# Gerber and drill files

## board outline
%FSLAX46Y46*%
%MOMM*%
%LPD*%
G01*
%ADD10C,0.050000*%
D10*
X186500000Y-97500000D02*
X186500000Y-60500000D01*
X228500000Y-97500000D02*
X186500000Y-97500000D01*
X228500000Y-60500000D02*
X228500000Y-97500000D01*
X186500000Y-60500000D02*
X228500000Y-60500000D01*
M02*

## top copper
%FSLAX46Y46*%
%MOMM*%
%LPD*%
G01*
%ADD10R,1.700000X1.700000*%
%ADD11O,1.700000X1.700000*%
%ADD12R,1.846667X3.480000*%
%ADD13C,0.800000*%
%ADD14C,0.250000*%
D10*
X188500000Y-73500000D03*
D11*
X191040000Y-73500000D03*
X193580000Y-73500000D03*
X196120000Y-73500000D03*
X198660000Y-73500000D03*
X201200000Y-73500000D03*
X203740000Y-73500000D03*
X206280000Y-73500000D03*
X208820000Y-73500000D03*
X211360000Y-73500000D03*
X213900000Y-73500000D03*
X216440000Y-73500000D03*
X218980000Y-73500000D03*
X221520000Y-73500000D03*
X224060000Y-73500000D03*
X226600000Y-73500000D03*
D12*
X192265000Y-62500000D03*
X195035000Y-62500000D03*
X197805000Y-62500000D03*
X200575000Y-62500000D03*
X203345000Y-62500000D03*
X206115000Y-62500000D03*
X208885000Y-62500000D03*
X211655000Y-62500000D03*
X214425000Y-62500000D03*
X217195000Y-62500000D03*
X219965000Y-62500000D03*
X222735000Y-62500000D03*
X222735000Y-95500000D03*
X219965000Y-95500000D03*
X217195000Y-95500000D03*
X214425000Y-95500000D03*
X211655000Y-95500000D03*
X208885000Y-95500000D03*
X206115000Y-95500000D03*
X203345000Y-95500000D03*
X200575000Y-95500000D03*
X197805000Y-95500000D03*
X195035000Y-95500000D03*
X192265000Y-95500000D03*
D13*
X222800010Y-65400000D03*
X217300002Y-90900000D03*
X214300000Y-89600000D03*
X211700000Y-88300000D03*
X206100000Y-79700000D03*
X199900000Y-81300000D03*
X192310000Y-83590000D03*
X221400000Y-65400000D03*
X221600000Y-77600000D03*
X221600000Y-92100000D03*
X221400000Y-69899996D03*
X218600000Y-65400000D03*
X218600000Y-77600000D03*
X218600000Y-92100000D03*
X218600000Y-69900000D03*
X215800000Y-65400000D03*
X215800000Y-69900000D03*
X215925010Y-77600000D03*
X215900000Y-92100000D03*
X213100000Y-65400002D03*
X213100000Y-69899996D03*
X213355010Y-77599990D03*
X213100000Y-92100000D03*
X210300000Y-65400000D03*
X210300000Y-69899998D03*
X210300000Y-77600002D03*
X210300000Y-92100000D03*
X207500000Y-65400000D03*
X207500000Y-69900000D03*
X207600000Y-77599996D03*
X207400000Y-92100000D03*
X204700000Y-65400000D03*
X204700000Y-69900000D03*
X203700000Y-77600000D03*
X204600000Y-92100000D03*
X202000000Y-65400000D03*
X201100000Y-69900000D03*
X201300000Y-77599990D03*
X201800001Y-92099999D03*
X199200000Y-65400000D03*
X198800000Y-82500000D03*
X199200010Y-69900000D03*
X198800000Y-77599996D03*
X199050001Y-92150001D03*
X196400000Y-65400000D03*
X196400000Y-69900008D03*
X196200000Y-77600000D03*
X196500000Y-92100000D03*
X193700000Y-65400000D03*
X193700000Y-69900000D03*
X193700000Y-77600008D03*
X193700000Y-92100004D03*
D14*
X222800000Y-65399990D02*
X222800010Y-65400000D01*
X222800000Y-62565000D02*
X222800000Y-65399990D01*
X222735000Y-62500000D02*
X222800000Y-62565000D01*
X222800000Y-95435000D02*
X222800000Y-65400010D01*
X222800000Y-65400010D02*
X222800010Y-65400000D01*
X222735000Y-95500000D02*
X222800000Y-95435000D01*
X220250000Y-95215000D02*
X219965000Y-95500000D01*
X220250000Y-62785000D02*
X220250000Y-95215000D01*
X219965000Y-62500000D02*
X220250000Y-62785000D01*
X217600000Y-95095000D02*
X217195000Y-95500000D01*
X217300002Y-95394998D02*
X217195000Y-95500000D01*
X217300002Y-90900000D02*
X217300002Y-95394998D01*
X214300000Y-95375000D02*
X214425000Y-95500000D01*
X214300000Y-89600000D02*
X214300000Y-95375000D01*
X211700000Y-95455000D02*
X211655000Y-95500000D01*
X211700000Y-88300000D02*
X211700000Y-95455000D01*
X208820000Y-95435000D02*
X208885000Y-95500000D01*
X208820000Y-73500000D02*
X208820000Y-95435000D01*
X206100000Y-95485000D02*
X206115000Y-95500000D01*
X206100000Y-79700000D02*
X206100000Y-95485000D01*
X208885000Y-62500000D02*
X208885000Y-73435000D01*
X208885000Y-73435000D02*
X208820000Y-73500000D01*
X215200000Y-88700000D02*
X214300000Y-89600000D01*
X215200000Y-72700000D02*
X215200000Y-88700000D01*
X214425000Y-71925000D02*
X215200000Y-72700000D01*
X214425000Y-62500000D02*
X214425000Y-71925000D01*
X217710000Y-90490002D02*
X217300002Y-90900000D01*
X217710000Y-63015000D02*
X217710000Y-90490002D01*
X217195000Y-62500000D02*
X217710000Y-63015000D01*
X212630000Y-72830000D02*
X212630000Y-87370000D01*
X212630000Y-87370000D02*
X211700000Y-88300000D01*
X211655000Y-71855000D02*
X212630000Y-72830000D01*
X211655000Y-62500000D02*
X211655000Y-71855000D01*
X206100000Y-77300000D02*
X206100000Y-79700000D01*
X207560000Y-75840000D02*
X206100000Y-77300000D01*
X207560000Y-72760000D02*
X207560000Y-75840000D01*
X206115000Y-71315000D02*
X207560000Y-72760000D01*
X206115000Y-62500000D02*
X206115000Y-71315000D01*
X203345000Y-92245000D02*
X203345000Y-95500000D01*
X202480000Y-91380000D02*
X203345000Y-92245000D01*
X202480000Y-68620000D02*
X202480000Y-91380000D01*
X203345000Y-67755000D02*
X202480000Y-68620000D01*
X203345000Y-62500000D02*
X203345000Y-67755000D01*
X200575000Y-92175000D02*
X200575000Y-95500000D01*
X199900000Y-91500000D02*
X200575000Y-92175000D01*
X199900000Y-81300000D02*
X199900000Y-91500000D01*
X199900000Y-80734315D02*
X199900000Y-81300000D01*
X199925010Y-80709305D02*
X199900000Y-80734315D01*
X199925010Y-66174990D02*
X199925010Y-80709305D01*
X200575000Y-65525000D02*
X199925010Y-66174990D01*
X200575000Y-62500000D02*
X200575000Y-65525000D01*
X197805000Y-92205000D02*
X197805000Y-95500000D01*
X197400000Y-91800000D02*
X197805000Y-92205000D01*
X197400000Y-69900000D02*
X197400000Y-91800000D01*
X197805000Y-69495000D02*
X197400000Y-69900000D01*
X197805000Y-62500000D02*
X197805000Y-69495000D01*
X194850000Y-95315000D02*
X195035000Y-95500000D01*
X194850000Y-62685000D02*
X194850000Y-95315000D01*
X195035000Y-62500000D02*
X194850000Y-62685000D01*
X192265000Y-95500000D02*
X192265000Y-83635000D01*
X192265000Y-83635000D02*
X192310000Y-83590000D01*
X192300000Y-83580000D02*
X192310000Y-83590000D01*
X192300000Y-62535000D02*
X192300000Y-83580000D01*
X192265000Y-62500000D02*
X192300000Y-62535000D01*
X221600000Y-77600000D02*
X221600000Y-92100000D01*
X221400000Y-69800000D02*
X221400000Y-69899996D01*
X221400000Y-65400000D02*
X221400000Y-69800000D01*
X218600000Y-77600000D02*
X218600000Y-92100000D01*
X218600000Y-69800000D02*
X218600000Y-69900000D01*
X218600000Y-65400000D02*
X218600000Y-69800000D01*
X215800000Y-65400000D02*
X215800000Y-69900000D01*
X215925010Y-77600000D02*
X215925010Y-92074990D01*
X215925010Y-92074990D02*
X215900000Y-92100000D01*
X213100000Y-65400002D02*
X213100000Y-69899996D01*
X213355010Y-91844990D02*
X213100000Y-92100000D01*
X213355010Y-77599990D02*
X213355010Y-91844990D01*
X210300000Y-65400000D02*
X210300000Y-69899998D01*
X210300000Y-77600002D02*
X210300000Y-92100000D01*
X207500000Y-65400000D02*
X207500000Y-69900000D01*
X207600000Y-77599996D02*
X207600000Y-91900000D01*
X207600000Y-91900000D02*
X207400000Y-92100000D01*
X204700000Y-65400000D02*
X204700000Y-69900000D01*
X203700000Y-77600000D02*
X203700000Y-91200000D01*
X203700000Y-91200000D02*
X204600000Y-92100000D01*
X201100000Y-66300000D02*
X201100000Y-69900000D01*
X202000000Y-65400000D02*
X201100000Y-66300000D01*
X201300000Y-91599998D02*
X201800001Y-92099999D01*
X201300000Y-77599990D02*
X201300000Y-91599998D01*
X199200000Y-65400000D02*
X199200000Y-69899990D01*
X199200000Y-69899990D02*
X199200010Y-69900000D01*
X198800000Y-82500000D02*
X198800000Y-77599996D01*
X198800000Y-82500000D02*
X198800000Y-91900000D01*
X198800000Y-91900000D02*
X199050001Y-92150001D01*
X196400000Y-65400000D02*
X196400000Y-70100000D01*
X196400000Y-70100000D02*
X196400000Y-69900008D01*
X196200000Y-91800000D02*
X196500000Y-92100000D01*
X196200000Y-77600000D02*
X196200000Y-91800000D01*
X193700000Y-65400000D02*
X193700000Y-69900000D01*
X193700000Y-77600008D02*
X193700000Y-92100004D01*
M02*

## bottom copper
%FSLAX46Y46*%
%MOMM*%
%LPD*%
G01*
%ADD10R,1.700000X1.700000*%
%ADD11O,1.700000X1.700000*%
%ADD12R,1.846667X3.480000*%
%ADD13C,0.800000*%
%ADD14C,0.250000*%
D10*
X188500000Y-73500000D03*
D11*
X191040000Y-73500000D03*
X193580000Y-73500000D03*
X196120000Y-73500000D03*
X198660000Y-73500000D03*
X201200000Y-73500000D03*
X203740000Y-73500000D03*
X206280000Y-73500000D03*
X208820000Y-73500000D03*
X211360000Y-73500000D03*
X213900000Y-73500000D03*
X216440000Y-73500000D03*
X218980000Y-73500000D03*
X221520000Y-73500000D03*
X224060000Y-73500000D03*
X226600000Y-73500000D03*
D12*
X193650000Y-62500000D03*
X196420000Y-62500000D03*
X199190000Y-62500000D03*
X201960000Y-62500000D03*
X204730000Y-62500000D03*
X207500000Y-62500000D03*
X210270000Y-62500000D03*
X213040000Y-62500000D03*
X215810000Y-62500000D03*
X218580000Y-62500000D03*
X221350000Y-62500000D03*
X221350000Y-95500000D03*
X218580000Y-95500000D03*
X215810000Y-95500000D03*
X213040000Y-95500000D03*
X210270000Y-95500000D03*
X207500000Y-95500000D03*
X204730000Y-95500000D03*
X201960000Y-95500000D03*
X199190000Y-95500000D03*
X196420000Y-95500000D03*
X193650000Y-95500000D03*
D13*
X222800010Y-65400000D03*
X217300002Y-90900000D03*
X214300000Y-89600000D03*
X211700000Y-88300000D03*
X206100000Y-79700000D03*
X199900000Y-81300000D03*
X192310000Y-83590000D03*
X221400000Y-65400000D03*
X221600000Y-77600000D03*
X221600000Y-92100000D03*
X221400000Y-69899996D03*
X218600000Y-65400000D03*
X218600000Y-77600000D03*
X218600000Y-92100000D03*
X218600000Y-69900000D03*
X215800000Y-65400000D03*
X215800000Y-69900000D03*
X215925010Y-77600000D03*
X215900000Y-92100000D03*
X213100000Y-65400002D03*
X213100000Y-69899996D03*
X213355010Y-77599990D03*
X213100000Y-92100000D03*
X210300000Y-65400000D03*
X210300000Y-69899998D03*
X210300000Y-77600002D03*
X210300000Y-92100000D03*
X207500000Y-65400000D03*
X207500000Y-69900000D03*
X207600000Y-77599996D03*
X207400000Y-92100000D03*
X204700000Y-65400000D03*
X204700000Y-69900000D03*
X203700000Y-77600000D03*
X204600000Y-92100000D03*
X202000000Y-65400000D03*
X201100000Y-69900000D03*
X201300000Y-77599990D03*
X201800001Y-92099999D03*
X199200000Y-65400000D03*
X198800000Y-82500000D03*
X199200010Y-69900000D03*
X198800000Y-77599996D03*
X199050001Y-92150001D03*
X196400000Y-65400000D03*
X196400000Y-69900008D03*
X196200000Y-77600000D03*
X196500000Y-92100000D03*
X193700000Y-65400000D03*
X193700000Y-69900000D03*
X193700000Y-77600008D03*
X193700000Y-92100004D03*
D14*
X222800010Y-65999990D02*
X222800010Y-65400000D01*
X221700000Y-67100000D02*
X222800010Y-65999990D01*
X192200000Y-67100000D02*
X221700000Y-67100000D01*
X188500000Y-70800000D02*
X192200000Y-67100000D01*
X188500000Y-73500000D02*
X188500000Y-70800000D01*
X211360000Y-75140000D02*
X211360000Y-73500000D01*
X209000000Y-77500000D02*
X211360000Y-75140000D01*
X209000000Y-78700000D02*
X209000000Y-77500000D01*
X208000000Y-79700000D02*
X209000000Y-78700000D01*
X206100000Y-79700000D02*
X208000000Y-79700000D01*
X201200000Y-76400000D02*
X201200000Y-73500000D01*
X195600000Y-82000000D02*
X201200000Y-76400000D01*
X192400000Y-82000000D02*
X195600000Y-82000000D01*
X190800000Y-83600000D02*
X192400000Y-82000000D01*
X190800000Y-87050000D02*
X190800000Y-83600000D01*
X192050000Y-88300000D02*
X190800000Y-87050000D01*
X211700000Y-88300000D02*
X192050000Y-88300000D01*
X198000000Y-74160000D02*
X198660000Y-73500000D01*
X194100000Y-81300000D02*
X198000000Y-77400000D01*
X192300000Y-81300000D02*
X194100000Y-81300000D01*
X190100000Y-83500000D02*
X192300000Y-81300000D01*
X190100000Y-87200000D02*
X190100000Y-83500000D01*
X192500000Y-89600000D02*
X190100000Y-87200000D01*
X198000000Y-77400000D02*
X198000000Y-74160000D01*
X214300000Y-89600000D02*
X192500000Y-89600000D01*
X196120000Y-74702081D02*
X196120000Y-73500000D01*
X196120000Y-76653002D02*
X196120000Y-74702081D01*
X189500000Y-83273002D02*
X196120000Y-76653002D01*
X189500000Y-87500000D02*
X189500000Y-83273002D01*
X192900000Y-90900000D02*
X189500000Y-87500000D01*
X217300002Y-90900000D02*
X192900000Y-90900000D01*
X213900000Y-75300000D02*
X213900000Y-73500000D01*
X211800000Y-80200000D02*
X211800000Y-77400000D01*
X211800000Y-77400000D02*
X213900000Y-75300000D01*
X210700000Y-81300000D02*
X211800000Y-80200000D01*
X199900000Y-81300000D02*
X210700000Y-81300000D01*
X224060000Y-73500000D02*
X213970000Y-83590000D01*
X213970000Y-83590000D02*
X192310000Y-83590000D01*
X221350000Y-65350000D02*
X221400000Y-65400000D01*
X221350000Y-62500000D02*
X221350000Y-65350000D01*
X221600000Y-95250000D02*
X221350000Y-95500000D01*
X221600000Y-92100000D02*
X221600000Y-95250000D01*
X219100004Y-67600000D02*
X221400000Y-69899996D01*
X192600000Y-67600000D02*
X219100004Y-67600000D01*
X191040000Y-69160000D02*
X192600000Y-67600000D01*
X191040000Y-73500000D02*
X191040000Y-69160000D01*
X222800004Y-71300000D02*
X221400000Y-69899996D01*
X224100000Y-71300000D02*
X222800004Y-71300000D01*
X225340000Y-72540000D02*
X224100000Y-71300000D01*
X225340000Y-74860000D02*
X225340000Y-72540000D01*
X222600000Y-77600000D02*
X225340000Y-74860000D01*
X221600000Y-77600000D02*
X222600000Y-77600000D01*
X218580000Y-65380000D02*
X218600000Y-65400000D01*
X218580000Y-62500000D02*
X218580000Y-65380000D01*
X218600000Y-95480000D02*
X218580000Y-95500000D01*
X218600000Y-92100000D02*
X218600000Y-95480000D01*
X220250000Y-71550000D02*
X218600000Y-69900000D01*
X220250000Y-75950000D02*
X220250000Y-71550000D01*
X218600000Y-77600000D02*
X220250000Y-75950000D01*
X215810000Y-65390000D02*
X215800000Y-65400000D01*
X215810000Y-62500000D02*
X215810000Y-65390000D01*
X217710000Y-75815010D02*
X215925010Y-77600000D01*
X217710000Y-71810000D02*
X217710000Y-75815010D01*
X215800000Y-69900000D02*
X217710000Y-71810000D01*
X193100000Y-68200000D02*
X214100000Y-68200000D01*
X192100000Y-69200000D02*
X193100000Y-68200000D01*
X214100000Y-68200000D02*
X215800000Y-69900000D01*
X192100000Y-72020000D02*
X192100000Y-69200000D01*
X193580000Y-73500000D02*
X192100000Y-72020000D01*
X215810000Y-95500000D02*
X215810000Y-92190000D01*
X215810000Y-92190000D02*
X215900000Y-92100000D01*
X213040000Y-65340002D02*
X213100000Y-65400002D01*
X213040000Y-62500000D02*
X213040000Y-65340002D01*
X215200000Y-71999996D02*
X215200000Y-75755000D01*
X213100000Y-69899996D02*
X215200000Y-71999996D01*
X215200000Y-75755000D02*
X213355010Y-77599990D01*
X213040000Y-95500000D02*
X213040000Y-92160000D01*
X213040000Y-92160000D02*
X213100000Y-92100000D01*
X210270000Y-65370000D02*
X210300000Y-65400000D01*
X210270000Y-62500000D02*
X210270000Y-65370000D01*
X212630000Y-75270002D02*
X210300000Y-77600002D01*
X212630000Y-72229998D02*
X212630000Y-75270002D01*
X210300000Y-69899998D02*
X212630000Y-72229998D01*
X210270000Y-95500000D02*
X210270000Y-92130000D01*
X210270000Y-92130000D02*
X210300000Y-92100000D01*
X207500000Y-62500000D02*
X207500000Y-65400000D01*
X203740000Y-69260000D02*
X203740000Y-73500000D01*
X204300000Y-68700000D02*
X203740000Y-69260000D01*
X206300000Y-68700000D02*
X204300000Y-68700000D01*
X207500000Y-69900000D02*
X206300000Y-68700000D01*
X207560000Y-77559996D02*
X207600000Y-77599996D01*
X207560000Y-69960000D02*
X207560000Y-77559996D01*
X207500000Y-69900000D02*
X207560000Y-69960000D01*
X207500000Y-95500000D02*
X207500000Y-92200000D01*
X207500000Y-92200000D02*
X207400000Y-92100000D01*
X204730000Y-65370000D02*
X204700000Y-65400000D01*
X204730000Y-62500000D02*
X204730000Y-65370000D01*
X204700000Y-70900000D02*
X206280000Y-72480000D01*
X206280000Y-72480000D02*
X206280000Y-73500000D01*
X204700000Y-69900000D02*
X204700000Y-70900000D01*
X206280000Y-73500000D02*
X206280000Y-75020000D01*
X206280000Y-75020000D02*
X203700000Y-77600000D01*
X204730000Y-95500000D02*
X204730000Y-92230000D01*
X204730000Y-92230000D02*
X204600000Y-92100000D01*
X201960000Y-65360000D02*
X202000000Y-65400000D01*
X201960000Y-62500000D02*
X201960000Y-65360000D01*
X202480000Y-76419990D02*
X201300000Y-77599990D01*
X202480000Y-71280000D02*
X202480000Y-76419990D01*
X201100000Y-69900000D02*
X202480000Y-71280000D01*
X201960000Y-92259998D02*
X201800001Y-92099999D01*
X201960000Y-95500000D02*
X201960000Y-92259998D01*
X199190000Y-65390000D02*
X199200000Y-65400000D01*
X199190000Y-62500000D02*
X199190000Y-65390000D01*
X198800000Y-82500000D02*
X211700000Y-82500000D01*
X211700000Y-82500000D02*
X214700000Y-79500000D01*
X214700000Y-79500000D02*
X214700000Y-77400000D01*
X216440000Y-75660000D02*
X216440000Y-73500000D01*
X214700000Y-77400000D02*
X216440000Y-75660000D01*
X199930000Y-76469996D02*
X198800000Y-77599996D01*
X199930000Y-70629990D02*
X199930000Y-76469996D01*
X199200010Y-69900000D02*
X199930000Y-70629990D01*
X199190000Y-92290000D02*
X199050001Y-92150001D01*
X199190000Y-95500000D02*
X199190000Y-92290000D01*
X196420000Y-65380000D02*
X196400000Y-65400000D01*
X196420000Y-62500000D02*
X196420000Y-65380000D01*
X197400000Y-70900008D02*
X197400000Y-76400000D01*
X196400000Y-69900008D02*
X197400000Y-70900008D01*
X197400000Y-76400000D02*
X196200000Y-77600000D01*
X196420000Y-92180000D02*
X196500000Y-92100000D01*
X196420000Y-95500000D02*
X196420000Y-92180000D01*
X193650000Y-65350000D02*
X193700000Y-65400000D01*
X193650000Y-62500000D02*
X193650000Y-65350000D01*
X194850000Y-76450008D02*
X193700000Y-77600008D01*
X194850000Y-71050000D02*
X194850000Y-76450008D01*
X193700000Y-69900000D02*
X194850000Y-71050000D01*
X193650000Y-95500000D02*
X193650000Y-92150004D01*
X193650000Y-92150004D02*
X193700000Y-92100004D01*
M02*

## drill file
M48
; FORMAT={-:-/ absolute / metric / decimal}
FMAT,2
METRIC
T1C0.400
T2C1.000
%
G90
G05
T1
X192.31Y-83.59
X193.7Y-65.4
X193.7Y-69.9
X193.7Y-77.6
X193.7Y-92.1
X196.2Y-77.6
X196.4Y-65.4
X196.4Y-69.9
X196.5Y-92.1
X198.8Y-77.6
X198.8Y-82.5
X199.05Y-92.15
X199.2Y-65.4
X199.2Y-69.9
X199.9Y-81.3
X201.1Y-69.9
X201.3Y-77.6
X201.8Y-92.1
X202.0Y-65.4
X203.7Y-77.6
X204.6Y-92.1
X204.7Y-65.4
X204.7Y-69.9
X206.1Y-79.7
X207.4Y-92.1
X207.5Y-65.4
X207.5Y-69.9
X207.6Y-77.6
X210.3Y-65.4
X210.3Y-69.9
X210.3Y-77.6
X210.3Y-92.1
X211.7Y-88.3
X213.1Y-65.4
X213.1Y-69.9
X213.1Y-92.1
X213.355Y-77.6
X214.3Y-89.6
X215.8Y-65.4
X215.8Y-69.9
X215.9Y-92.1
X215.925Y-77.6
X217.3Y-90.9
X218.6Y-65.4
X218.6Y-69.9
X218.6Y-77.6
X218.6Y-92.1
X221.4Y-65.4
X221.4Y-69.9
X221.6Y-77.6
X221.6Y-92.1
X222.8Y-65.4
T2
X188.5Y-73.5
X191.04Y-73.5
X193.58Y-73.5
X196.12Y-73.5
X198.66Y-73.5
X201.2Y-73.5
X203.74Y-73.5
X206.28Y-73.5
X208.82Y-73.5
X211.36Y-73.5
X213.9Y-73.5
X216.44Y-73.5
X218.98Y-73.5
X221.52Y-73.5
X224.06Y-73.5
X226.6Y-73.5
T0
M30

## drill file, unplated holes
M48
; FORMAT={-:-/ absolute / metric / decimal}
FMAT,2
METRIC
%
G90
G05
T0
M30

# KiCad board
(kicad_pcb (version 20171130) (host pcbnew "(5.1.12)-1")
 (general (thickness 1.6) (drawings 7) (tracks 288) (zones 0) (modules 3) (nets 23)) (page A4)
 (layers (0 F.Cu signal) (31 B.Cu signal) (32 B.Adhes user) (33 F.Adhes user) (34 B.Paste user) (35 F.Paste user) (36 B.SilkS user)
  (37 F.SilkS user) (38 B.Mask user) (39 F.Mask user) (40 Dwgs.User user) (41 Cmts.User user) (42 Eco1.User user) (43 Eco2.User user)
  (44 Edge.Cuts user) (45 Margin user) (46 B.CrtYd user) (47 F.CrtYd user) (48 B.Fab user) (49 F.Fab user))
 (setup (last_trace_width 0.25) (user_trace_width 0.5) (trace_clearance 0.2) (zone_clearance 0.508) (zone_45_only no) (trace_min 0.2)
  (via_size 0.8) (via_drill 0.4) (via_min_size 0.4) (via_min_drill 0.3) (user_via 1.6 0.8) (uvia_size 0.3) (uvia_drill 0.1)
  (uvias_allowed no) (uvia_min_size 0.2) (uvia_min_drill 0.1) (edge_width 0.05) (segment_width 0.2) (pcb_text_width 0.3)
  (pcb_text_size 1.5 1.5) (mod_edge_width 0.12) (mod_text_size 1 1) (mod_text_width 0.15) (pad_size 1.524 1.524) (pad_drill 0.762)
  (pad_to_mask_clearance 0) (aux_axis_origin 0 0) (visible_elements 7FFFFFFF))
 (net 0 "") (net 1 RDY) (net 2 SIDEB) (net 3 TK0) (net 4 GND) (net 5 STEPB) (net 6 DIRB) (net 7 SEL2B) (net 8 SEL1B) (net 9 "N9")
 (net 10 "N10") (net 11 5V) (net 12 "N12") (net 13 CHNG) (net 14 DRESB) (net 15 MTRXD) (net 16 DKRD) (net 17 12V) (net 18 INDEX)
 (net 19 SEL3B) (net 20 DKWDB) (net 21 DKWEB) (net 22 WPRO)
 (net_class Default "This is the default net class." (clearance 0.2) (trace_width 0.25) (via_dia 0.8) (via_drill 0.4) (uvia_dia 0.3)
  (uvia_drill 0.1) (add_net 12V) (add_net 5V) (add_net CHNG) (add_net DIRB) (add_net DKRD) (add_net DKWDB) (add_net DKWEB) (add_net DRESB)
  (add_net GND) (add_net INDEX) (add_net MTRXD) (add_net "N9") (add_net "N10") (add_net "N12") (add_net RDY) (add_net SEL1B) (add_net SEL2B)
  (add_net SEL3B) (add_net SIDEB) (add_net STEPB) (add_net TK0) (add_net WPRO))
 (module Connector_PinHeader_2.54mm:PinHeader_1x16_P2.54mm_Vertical (layer F.Cu) (at 188.5 73.5 90)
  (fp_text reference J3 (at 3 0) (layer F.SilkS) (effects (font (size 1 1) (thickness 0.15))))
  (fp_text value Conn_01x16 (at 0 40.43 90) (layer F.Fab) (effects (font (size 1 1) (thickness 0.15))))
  (pad 1 thru_hole rect (at 0 0 90) (size 1.7 1.7) (drill 1) (layers *.Cu *.Mask) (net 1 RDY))
  (pad 2 thru_hole oval (at 0 2.54 90) (size 1.7 1.7) (drill 1) (layers *.Cu *.Mask) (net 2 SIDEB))
  (pad 3 thru_hole oval (at 0 5.08 90) (size 1.7 1.7) (drill 1) (layers *.Cu *.Mask) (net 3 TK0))
  (pad 4 thru_hole oval (at 0 7.62 90) (size 1.7 1.7) (drill 1) (layers *.Cu *.Mask) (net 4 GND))
  (pad 5 thru_hole oval (at 0 10.16 90) (size 1.7 1.7) (drill 1) (layers *.Cu *.Mask) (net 4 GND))
  (pad 6 thru_hole oval (at 0 12.7 90) (size 1.7 1.7) (drill 1) (layers *.Cu *.Mask) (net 4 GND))
  (pad 7 thru_hole oval (at 0 15.24 90) (size 1.7 1.7) (drill 1) (layers *.Cu *.Mask) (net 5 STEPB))
  (pad 8 thru_hole oval (at 0 17.78 90) (size 1.7 1.7) (drill 1) (layers *.Cu *.Mask) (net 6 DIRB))
  (pad 9 thru_hole oval (at 0 20.32 90) (size 1.7 1.7) (drill 1) (layers *.Cu *.Mask) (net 4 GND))
  (pad 10 thru_hole oval (at 0 22.86 90) (size 1.7 1.7) (drill 1) (layers *.Cu *.Mask) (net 4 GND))
  (pad 11 thru_hole oval (at 0 25.4 90) (size 1.7 1.7) (drill 1) (layers *.Cu *.Mask) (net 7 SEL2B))
  (pad 12 thru_hole oval (at 0 27.94 90) (size 1.7 1.7) (drill 1) (layers *.Cu *.Mask) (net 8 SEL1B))
  (pad 13 thru_hole oval (at 0 30.48 90) (size 1.7 1.7) (drill 1) (layers *.Cu *.Mask) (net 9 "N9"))
  (pad 14 thru_hole oval (at 0 33.02 90) (size 1.7 1.7) (drill 1) (layers *.Cu *.Mask) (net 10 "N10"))
  (pad 15 thru_hole oval (at 0 35.56 90) (size 1.7 1.7) (drill 1) (layers *.Cu *.Mask) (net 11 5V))
  (pad 16 thru_hole oval (at 0 38.1 90) (size 1.7 1.7) (drill 1) (layers *.Cu *.Mask) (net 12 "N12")))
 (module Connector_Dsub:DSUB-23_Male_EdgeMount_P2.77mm (layer F.Cu) (at 207.5 62.5 180)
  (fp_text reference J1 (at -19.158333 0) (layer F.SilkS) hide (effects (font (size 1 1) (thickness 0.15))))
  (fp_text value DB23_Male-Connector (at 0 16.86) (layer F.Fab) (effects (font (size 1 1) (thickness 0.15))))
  (pad 12 smd rect (at 15.235 0 180) (size 1.846667 3.48) (layers F.Cu F.Paste F.Mask) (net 11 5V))
  (pad 11 smd rect (at 12.465 0 180) (size 1.846667 3.48) (layers F.Cu F.Paste F.Mask) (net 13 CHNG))
  (pad 10 smd rect (at 9.695 0 180) (size 1.846667 3.48) (layers F.Cu F.Paste F.Mask) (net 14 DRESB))
  (pad 9 smd rect (at 6.925 0 180) (size 1.846667 3.48) (layers F.Cu F.Paste F.Mask) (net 7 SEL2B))
  (pad 8 smd rect (at 4.155 0 180) (size 1.846667 3.48) (layers F.Cu F.Paste F.Mask) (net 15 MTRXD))
  (pad 7 smd rect (at 1.385 0 180) (size 1.846667 3.48) (layers F.Cu F.Paste F.Mask) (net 4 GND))
  (pad 6 smd rect (at -1.385 0 180) (size 1.846667 3.48) (layers F.Cu F.Paste F.Mask) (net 4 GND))
  (pad 5 smd rect (at -4.155 0 180) (size 1.846667 3.48) (layers F.Cu F.Paste F.Mask) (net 4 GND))
  (pad 4 smd rect (at -6.925 0 180) (size 1.846667 3.48) (layers F.Cu F.Paste F.Mask) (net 4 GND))
  (pad 3 smd rect (at -9.695 0 180) (size 1.846667 3.48) (layers F.Cu F.Paste F.Mask) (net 4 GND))
  (pad 2 smd rect (at -12.465 0 180) (size 1.846667 3.48) (layers F.Cu F.Paste F.Mask) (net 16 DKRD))
  (pad 1 smd rect (at -15.235 0 180) (size 1.846667 3.48) (layers F.Cu F.Paste F.Mask) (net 1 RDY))
  (pad 23 smd rect (at 13.85 0 180) (size 1.846667 3.48) (layers B.Cu B.Paste B.Mask) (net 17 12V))
  (pad 22 smd rect (at 11.08 0 180) (size 1.846667 3.48) (layers B.Cu B.Paste B.Mask) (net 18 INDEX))
  (pad 21 smd rect (at 8.31 0 180) (size 1.846667 3.48) (layers B.Cu B.Paste B.Mask) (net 8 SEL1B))
  (pad 20 smd rect (at 5.54 0 180) (size 1.846667 3.48) (layers B.Cu B.Paste B.Mask) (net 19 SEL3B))
  (pad 19 smd rect (at 2.77 0 180) (size 1.846667 3.48) (layers B.Cu B.Paste B.Mask) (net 6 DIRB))
  (pad 18 smd rect (at 0 0 180) (size 1.846667 3.48) (layers B.Cu B.Paste B.Mask) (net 5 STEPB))
  (pad 17 smd rect (at -2.77 0 180) (size 1.846667 3.48) (layers B.Cu B.Paste B.Mask) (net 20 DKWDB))
  (pad 16 smd rect (at -5.54 0 180) (size 1.846667 3.48) (layers B.Cu B.Paste B.Mask) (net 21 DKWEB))
  (pad 15 smd rect (at -8.31 0 180) (size 1.846667 3.48) (layers B.Cu B.Paste B.Mask) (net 3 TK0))
  (pad 14 smd rect (at -11.08 0 180) (size 1.846667 3.48) (layers B.Cu B.Paste B.Mask) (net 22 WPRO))
  (pad 13 smd rect (at -13.85 0 180) (size 1.846667 3.48) (layers B.Cu B.Paste B.Mask) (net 2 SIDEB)))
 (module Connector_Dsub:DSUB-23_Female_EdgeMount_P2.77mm (layer F.Cu) (at 207.5 95.5)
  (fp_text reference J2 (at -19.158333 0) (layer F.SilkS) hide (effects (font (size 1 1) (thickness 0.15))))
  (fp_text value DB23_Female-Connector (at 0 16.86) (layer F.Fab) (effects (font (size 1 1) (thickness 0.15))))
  (pad 1 smd rect (at 15.235 0) (size 1.846667 3.48) (layers F.Cu F.Paste F.Mask) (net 1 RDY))
  (pad 2 smd rect (at 12.465 0) (size 1.846667 3.48) (layers F.Cu F.Paste F.Mask) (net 16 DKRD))
  (pad 3 smd rect (at 9.695 0) (size 1.846667 3.48) (layers F.Cu F.Paste F.Mask) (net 4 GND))
  (pad 4 smd rect (at 6.925 0) (size 1.846667 3.48) (layers F.Cu F.Paste F.Mask) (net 4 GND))
  (pad 5 smd rect (at 4.155 0) (size 1.846667 3.48) (layers F.Cu F.Paste F.Mask) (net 4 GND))
  (pad 6 smd rect (at 1.385 0) (size 1.846667 3.48) (layers F.Cu F.Paste F.Mask) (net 4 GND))
  (pad 7 smd rect (at -1.385 0) (size 1.846667 3.48) (layers F.Cu F.Paste F.Mask) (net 4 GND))
  (pad 8 smd rect (at -4.155 0) (size 1.846667 3.48) (layers F.Cu F.Paste F.Mask) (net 15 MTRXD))
  (pad 9 smd rect (at -6.925 0) (size 1.846667 3.48) (layers F.Cu F.Paste F.Mask) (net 7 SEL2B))
  (pad 10 smd rect (at -9.695 0) (size 1.846667 3.48) (layers F.Cu F.Paste F.Mask) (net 14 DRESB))
  (pad 11 smd rect (at -12.465 0) (size 1.846667 3.48) (layers F.Cu F.Paste F.Mask) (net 13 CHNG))
  (pad 12 smd rect (at -15.235 0) (size 1.846667 3.48) (layers F.Cu F.Paste F.Mask) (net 11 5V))
  (pad 13 smd rect (at 13.85 0) (size 1.846667 3.48) (layers B.Cu B.Paste B.Mask) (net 2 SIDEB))
  (pad 14 smd rect (at 11.08 0) (size 1.846667 3.48) (layers B.Cu B.Paste B.Mask) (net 22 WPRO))
  (pad 15 smd rect (at 8.31 0) (size 1.846667 3.48) (layers B.Cu B.Paste B.Mask) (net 3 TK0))
  (pad 16 smd rect (at 5.54 0) (size 1.846667 3.48) (layers B.Cu B.Paste B.Mask) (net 21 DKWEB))
  (pad 17 smd rect (at 2.77 0) (size 1.846667 3.48) (layers B.Cu B.Paste B.Mask) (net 20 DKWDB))
  (pad 18 smd rect (at 0 0) (size 1.846667 3.48) (layers B.Cu B.Paste B.Mask) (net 5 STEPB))
  (pad 19 smd rect (at -2.77 0) (size 1.846667 3.48) (layers B.Cu B.Paste B.Mask) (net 6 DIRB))
  (pad 20 smd rect (at -5.54 0) (size 1.846667 3.48) (layers B.Cu B.Paste B.Mask) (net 19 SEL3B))
  (pad 21 smd rect (at -8.31 0) (size 1.846667 3.48) (layers B.Cu B.Paste B.Mask) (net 8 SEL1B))
  (pad 22 smd rect (at -11.08 0) (size 1.846667 3.48) (layers B.Cu B.Paste B.Mask) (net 18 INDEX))
  (pad 23 smd rect (at -13.85 0) (size 1.846667 3.48) (layers B.Cu B.Paste B.Mask) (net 17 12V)))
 (gr_line (start 186.5 97.5) (end 186.5 60.5) (layer Edge.Cuts) (width 0.05))
 (gr_line (start 228.5 97.5) (end 186.5 97.5) (layer Edge.Cuts) (width 0.05))
 (gr_line (start 228.5 60.5) (end 228.5 97.5) (layer Edge.Cuts) (width 0.05))
 (gr_line (start 186.5 60.5) (end 228.5 60.5) (layer Edge.Cuts) (width 0.05))
 (via (at 222.80001 65.4) (size 0.8) (drill 0.4) (layers F.Cu B.Cu) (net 1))
 (segment (start 222.8 65.39999) (end 222.80001 65.4) (width 0.25) (layer F.Cu) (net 1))
 (segment (start 222.8 62.565) (end 222.8 65.39999) (width 0.25) (layer F.Cu) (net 1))
 (segment (start 222.735 62.5) (end 222.8 62.565) (width 0.25) (layer F.Cu) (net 1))
 (segment (start 222.80001 65.99999) (end 222.80001 65.4) (width 0.25) (layer B.Cu) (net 1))
 (segment (start 221.7 67.1) (end 222.80001 65.99999) (width 0.25) (layer B.Cu) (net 1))
 (segment (start 192.2 67.1) (end 221.7 67.1) (width 0.25) (layer B.Cu) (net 1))
 (segment (start 188.5 70.8) (end 192.2 67.1) (width 0.25) (layer B.Cu) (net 1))
 (segment (start 188.5 73.5) (end 188.5 70.8) (width 0.25) (layer B.Cu) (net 1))
 (segment (start 222.8 95.435) (end 222.8 65.40001) (width 0.25) (layer F.Cu) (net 1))
 (segment (start 222.8 65.40001) (end 222.80001 65.4) (width 0.25) (layer F.Cu) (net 1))
 (segment (start 222.735 95.5) (end 222.8 95.435) (width 0.25) (layer F.Cu) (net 1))
 (segment (start 220.25 95.215) (end 219.965 95.5) (width 0.25) (layer F.Cu) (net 16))
 (segment (start 220.25 62.785) (end 220.25 95.215) (width 0.25) (layer F.Cu) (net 16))
 (segment (start 219.965 62.5) (end 220.25 62.785) (width 0.25) (layer F.Cu) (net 16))
 (segment (start 217.6 95.095) (end 217.195 95.5) (width 0.25) (layer F.Cu) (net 4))
 (via (at 217.300002 90.9) (size 0.8) (drill 0.4) (layers F.Cu B.Cu) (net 4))
 (segment (start 217.300002 95.394998) (end 217.195 95.5) (width 0.25) (layer F.Cu) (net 4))
 (segment (start 217.300002 90.9) (end 217.300002 95.394998) (width 0.25) (layer F.Cu) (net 4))
 (via (at 214.3 89.6) (size 0.8) (drill 0.4) (layers F.Cu B.Cu) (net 4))
 (segment (start 214.3 95.375) (end 214.425 95.5) (width 0.25) (layer F.Cu) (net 4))
 (segment (start 214.3 89.6) (end 214.3 95.375) (width 0.25) (layer F.Cu) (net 4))
 (via (at 211.7 88.3) (size 0.8) (drill 0.4) (layers F.Cu B.Cu) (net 4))
 (segment (start 211.7 95.455) (end 211.655 95.5) (width 0.25) (layer F.Cu) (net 4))
 (segment (start 211.7 88.3) (end 211.7 95.455) (width 0.25) (layer F.Cu) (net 4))
 (segment (start 208.82 95.435) (end 208.885 95.5) (width 0.25) (layer F.Cu) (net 4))
 (segment (start 208.82 73.5) (end 208.82 95.435) (width 0.25) (layer F.Cu) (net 4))
 (via (at 206.1 79.7) (size 0.8) (drill 0.4) (layers F.Cu B.Cu) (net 4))
 (segment (start 206.1 95.485) (end 206.115 95.5) (width 0.25) (layer F.Cu) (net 4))
 (segment (start 206.1 79.7) (end 206.1 95.485) (width 0.25) (layer F.Cu) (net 4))
 (segment (start 211.36 75.14) (end 211.36 73.5) (width 0.25) (layer B.Cu) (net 4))
 (segment (start 209 77.5) (end 211.36 75.14) (width 0.25) (layer B.Cu) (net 4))
 (segment (start 209 78.7) (end 209 77.5) (width 0.25) (layer B.Cu) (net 4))
 (segment (start 208 79.7) (end 209 78.7) (width 0.25) (layer B.Cu) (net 4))
 (segment (start 206.1 79.7) (end 208 79.7) (width 0.25) (layer B.Cu) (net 4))
 (segment (start 208.885 62.5) (end 208.885 73.435) (width 0.25) (layer F.Cu) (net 4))
 (segment (start 208.885 73.435) (end 208.82 73.5) (width 0.25) (layer F.Cu) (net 4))
 (segment (start 215.2 88.7) (end 214.3 89.6) (width 0.25) (layer F.Cu) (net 4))
 (segment (start 215.2 72.7) (end 215.2 88.7) (width 0.25) (layer F.Cu) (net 4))
 (segment (start 214.425 71.925) (end 215.2 72.7) (width 0.25) (layer F.Cu) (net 4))
 (segment (start 214.425 62.5) (end 214.425 71.925) (width 0.25) (layer F.Cu) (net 4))
 (segment (start 217.71 90.490002) (end 217.300002 90.9) (width 0.25) (layer F.Cu) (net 4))
 (segment (start 217.71 63.015) (end 217.71 90.490002) (width 0.25) (layer F.Cu) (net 4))
 (segment (start 217.195 62.5) (end 217.71 63.015) (width 0.25) (layer F.Cu) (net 4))
 (segment (start 212.63 72.83) (end 212.63 87.37) (width 0.25) (layer F.Cu) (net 4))
 (segment (start 212.63 87.37) (end 211.7 88.3) (width 0.25) (layer F.Cu) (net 4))
 (segment (start 211.655 71.855) (end 212.63 72.83) (width 0.25) (layer F.Cu) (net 4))
 (segment (start 211.655 62.5) (end 211.655 71.855) (width 0.25) (layer F.Cu) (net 4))
 (segment (start 206.1 77.3) (end 206.1 79.7) (width 0.25) (layer F.Cu) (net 4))
 (segment (start 207.56 75.84) (end 206.1 77.3) (width 0.25) (layer F.Cu) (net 4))
 (segment (start 207.56 72.76) (end 207.56 75.84) (width 0.25) (layer F.Cu) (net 4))
 (segment (start 206.115 71.315) (end 207.56 72.76) (width 0.25) (layer F.Cu) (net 4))
 (segment (start 206.115 62.5) (end 206.115 71.315) (width 0.25) (layer F.Cu) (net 4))
 (segment (start 201.2 76.4) (end 201.2 73.5) (width 0.25) (layer B.Cu) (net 4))
 (segment (start 195.6 82) (end 201.2 76.4) (width 0.25) (layer B.Cu) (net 4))
 (segment (start 192.4 82) (end 195.6 82) (width 0.25) (layer B.Cu) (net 4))
 (segment (start 190.8 83.6) (end 192.4 82) (width 0.25) (layer B.Cu) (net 4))
 (segment (start 190.8 87.05) (end 190.8 83.6) (width 0.25) (layer B.Cu) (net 4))
 (segment (start 192.05 88.3) (end 190.8 87.05) (width 0.25) (layer B.Cu) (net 4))
 (segment (start 211.7 88.3) (end 192.05 88.3) (width 0.25) (layer B.Cu) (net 4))
 (segment (start 198 74.16) (end 198.66 73.5) (width 0.25) (layer B.Cu) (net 4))
 (segment (start 194.1 81.3) (end 198 77.4) (width 0.25) (layer B.Cu) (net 4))
 (segment (start 192.3 81.3) (end 194.1 81.3) (width 0.25) (layer B.Cu) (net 4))
 (segment (start 190.1 83.5) (end 192.3 81.3) (width 0.25) (layer B.Cu) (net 4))
 (segment (start 190.1 87.2) (end 190.1 83.5) (width 0.25) (layer B.Cu) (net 4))
 (segment (start 192.5 89.6) (end 190.1 87.2) (width 0.25) (layer B.Cu) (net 4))
 (segment (start 198 77.4) (end 198 74.16) (width 0.25) (layer B.Cu) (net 4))
 (segment (start 214.3 89.6) (end 192.5 89.6) (width 0.25) (layer B.Cu) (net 4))
 (segment (start 196.12 74.702081) (end 196.12 73.5) (width 0.25) (layer B.Cu) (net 4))
 (segment (start 196.12 76.653002) (end 196.12 74.702081) (width 0.25) (layer B.Cu) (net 4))
 (segment (start 189.5 83.273002) (end 196.12 76.653002) (width 0.25) (layer B.Cu) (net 4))
 (segment (start 189.5 87.5) (end 189.5 83.273002) (width 0.25) (layer B.Cu) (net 4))
 (segment (start 192.9 90.9) (end 189.5 87.5) (width 0.25) (layer B.Cu) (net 4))
 (segment (start 217.300002 90.9) (end 192.9 90.9) (width 0.25) (layer B.Cu) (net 4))
 (segment (start 203.345 92.245) (end 203.345 95.5) (width 0.25) (layer F.Cu) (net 15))
 (segment (start 202.48 91.38) (end 203.345 92.245) (width 0.25) (layer F.Cu) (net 15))
 (segment (start 202.48 68.62) (end 202.48 91.38) (width 0.25) (layer F.Cu) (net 15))
 (segment (start 203.345 67.755) (end 202.48 68.62) (width 0.25) (layer F.Cu) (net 15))
 (segment (start 203.345 62.5) (end 203.345 67.755) (width 0.25) (layer F.Cu) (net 15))
 (via (at 199.9 81.3) (size 0.8) (drill 0.4) (layers F.Cu B.Cu) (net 7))
 (segment (start 213.9 75.3) (end 213.9 73.5) (width 0.25) (layer B.Cu) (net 7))
 (segment (start 211.8 80.2) (end 211.8 77.4) (width 0.25) (layer B.Cu) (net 7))
 (segment (start 211.8 77.4) (end 213.9 75.3) (width 0.25) (layer B.Cu) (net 7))
 (segment (start 210.7 81.3) (end 211.8 80.2) (width 0.25) (layer B.Cu) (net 7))
 (segment (start 199.9 81.3) (end 210.7 81.3) (width 0.25) (layer B.Cu) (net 7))
 (segment (start 200.575 92.175) (end 200.575 95.5) (width 0.25) (layer F.Cu) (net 7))
 (segment (start 199.9 91.5) (end 200.575 92.175) (width 0.25) (layer F.Cu) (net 7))
 (segment (start 199.9 81.3) (end 199.9 91.5) (width 0.25) (layer F.Cu) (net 7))
 (segment (start 199.9 80.734315) (end 199.9 81.3) (width 0.25) (layer F.Cu) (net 7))
 (segment (start 199.92501 80.709305) (end 199.9 80.734315) (width 0.25) (layer F.Cu) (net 7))
 (segment (start 199.92501 66.17499) (end 199.92501 80.709305) (width 0.25) (layer F.Cu) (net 7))
 (segment (start 200.575 65.525) (end 199.92501 66.17499) (width 0.25) (layer F.Cu) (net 7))
 (segment (start 200.575 62.5) (end 200.575 65.525) (width 0.25) (layer F.Cu) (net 7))
 (segment (start 197.805 92.205) (end 197.805 95.5) (width 0.25) (layer F.Cu) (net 14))
 (segment (start 197.4 91.8) (end 197.805 92.205) (width 0.25) (layer F.Cu) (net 14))
 (segment (start 197.4 69.9) (end 197.4 91.8) (width 0.25) (layer F.Cu) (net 14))
 (segment (start 197.805 69.495) (end 197.4 69.9) (width 0.25) (layer F.Cu) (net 14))
 (segment (start 197.805 62.5) (end 197.805 69.495) (width 0.25) (layer F.Cu) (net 14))
 (segment (start 194.85 95.315) (end 195.035 95.5) (width 0.25) (layer F.Cu) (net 13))
 (segment (start 194.85 62.685) (end 194.85 95.315) (width 0.25) (layer F.Cu) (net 13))
 (segment (start 195.035 62.5) (end 194.85 62.685) (width 0.25) (layer F.Cu) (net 13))
 (via (at 192.31 83.59) (size 0.8) (drill 0.4) (layers F.Cu B.Cu) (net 11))
 (segment (start 224.06 73.5) (end 213.97 83.59) (width 0.25) (layer B.Cu) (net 11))
 (segment (start 192.265 95.5) (end 192.265 83.635) (width 0.25) (layer F.Cu) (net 11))
 (segment (start 213.97 83.59) (end 192.31 83.59) (width 0.25) (layer B.Cu) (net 11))
 (segment (start 192.265 83.635) (end 192.31 83.59) (width 0.25) (layer F.Cu) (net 11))
 (segment (start 192.3 83.58) (end 192.31 83.59) (width 0.25) (layer F.Cu) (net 11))
 (segment (start 192.3 62.535) (end 192.3 83.58) (width 0.25) (layer F.Cu) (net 11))
 (segment (start 192.265 62.5) (end 192.3 62.535) (width 0.25) (layer F.Cu) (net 11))
 (via (at 221.4 65.4) (size 0.8) (drill 0.4) (layers F.Cu B.Cu) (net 2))
 (segment (start 221.35 65.35) (end 221.4 65.4) (width 0.25) (layer B.Cu) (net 2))
 (segment (start 221.35 62.5) (end 221.35 65.35) (width 0.25) (layer B.Cu) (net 2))
 (via (at 221.6 77.6) (size 0.8) (drill 0.4) (layers F.Cu B.Cu) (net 2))
 (via (at 221.6 92.1) (size 0.8) (drill 0.4) (layers F.Cu B.Cu) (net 2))
 (segment (start 221.6 77.6) (end 221.6 92.1) (width 0.25) (layer F.Cu) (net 2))
 (segment (start 221.6 95.25) (end 221.35 95.5) (width 0.25) (layer B.Cu) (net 2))
 (segment (start 221.6 92.1) (end 221.6 95.25) (width 0.25) (layer B.Cu) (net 2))
 (via (at 221.4 69.899996) (size 0.8) (drill 0.4) (layers F.Cu B.Cu) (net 2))
 (segment (start 221.4 69.8) (end 221.4 69.899996) (width 0.25) (layer F.Cu) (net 2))
 (segment (start 221.4 65.4) (end 221.4 69.8) (width 0.25) (layer F.Cu) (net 2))
 (segment (start 219.100004 67.6) (end 221.4 69.899996) (width 0.25) (layer B.Cu) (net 2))
 (segment (start 192.6 67.6) (end 219.100004 67.6) (width 0.25) (layer B.Cu) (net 2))
 (segment (start 191.04 69.16) (end 192.6 67.6) (width 0.25) (layer B.Cu) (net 2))
 (segment (start 191.04 73.5) (end 191.04 69.16) (width 0.25) (layer B.Cu) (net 2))
 (segment (start 222.800004 71.3) (end 221.4 69.899996) (width 0.25) (layer B.Cu) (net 2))
 (segment (start 224.1 71.3) (end 222.800004 71.3) (width 0.25) (layer B.Cu) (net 2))
 (segment (start 225.34 72.54) (end 224.1 71.3) (width 0.25) (layer B.Cu) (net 2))
 (segment (start 225.34 74.86) (end 225.34 72.54) (width 0.25) (layer B.Cu) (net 2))
 (segment (start 222.6 77.6) (end 225.34 74.86) (width 0.25) (layer B.Cu) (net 2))
 (segment (start 221.6 77.6) (end 222.6 77.6) (width 0.25) (layer B.Cu) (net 2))
 (via (at 218.6 65.4) (size 0.8) (drill 0.4) (layers F.Cu B.Cu) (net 22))
 (segment (start 218.58 65.38) (end 218.6 65.4) (width 0.25) (layer B.Cu) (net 22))
 (segment (start 218.58 62.5) (end 218.58 65.38) (width 0.25) (layer B.Cu) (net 22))
 (via (at 218.6 77.6) (size 0.8) (drill 0.4) (layers F.Cu B.Cu) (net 22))
 (via (at 218.6 92.1) (size 0.8) (drill 0.4) (layers F.Cu B.Cu) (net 22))
 (segment (start 218.6 77.6) (end 218.6 92.1) (width 0.25) (layer F.Cu) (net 22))
 (segment (start 218.6 95.48) (end 218.58 95.5) (width 0.25) (layer B.Cu) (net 22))
 (segment (start 218.6 92.1) (end 218.6 95.48) (width 0.25) (layer B.Cu) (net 22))
 (via (at 218.6 69.9) (size 0.8) (drill 0.4) (layers F.Cu B.Cu) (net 22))
 (segment (start 218.6 69.8) (end 218.6 69.9) (width 0.25) (layer F.Cu) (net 22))
 (segment (start 218.6 65.4) (end 218.6 69.8) (width 0.25) (layer F.Cu) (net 22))
 (segment (start 220.25 71.55) (end 218.6 69.9) (width 0.25) (layer B.Cu) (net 22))
 (segment (start 220.25 75.95) (end 220.25 71.55) (width 0.25) (layer B.Cu) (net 22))
 (segment (start 218.6 77.6) (end 220.25 75.95) (width 0.25) (layer B.Cu) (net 22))
 (via (at 215.8 65.4) (size 0.8) (drill 0.4) (layers F.Cu B.Cu) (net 3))
 (segment (start 215.81 65.39) (end 215.8 65.4) (width 0.25) (layer B.Cu) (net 3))
 (segment (start 215.81 62.5) (end 215.81 65.39) (width 0.25) (layer B.Cu) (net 3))
 (via (at 215.8 69.9) (size 0.8) (drill 0.4) (layers F.Cu B.Cu) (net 3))
 (segment (start 215.8 65.4) (end 215.8 69.9) (width 0.25) (layer F.Cu) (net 3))
 (via (at 215.92501 77.6) (size 0.8) (drill 0.4) (layers F.Cu B.Cu) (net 3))
 (segment (start 217.71 75.81501) (end 215.92501 77.6) (width 0.25) (layer B.Cu) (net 3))
 (segment (start 217.71 71.81) (end 217.71 75.81501) (width 0.25) (layer B.Cu) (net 3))
 (segment (start 215.8 69.9) (end 217.71 71.81) (width 0.25) (layer B.Cu) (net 3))
 (segment (start 193.1 68.2) (end 214.1 68.2) (width 0.25) (layer B.Cu) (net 3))
 (segment (start 192.1 69.2) (end 193.1 68.2) (width 0.25) (layer B.Cu) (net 3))
 (segment (start 214.1 68.2) (end 215.8 69.9) (width 0.25) (layer B.Cu) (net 3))
 (segment (start 192.1 72.02) (end 192.1 69.2) (width 0.25) (layer B.Cu) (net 3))
 (segment (start 193.58 73.5) (end 192.1 72.02) (width 0.25) (layer B.Cu) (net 3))
 (via (at 215.9 92.1) (size 0.8) (drill 0.4) (layers F.Cu B.Cu) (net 3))
 (segment (start 215.81 95.5) (end 215.81 92.19) (width 0.25) (layer B.Cu) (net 3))
 (segment (start 215.81 92.19) (end 215.9 92.1) (width 0.25) (layer B.Cu) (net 3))
 (segment (start 215.92501 77.6) (end 215.92501 92.07499) (width 0.25) (layer F.Cu) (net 3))
 (segment (start 215.92501 92.07499) (end 215.9 92.1) (width 0.25) (layer F.Cu) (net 3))
 (segment (start 213.04 65.340002) (end 213.1 65.400002) (width 0.25) (layer B.Cu) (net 21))
 (via (at 213.1 65.400002) (size 0.8) (drill 0.4) (layers F.Cu B.Cu) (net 21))
 (segment (start 213.04 62.5) (end 213.04 65.340002) (width 0.25) (layer B.Cu) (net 21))
 (segment (start 213.1 65.400002) (end 213.1 69.899996) (width 0.25) (layer F.Cu) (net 21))
 (via (at 213.1 69.899996) (size 0.8) (drill 0.4) (layers F.Cu B.Cu) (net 21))
 (segment (start 215.2 71.999996) (end 215.2 75.755) (width 0.25) (layer B.Cu) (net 21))
 (via (at 213.35501 77.59999) (size 0.8) (drill 0.4) (layers F.Cu B.Cu) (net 21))
 (segment (start 213.1 69.899996) (end 215.2 71.999996) (width 0.25) (layer B.Cu) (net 21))
 (segment (start 215.2 75.755) (end 213.35501 77.59999) (width 0.25) (layer B.Cu) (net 21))
 (via (at 213.1 92.1) (size 0.8) (drill 0.4) (layers F.Cu B.Cu) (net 21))
 (segment (start 213.35501 91.84499) (end 213.1 92.1) (width 0.25) (layer F.Cu) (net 21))
 (segment (start 213.04 95.5) (end 213.04 92.16) (width 0.25) (layer B.Cu) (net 21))
 (segment (start 213.04 92.16) (end 213.1 92.1) (width 0.25) (layer B.Cu) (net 21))
 (segment (start 213.35501 77.59999) (end 213.35501 91.84499) (width 0.25) (layer F.Cu) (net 21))
 (via (at 210.3 65.4) (size 0.8) (drill 0.4) (layers F.Cu B.Cu) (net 20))
 (segment (start 210.27 65.37) (end 210.3 65.4) (width 0.25) (layer B.Cu) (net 20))
 (segment (start 210.27 62.5) (end 210.27 65.37) (width 0.25) (layer B.Cu) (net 20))
 (segment (start 210.3 65.4) (end 210.3 69.899998) (width 0.25) (layer F.Cu) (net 20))
 (via (at 210.3 69.899998) (size 0.8) (drill 0.4) (layers F.Cu B.Cu) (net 20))
 (via (at 210.3 77.600002) (size 0.8) (drill 0.4) (layers F.Cu B.Cu) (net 20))
 (segment (start 212.63 75.270002) (end 210.3 77.600002) (width 0.25) (layer B.Cu) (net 20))
 (segment (start 212.63 72.229998) (end 212.63 75.270002) (width 0.25) (layer B.Cu) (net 20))
 (segment (start 210.3 69.899998) (end 212.63 72.229998) (width 0.25) (layer B.Cu) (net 20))
 (via (at 210.3 92.1) (size 0.8) (drill 0.4) (layers F.Cu B.Cu) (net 20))
 (segment (start 210.3 77.600002) (end 210.3 92.1) (width 0.25) (layer F.Cu) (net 20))
 (segment (start 210.27 95.5) (end 210.27 92.13) (width 0.25) (layer B.Cu) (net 20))
 (segment (start 210.27 92.13) (end 210.3 92.1) (width 0.25) (layer B.Cu) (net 20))
 (via (at 207.5 65.4) (size 0.8) (drill 0.4) (layers F.Cu B.Cu) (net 5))
 (segment (start 207.5 62.5) (end 207.5 65.4) (width 0.25) (layer B.Cu) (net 5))
 (via (at 207.5 69.9) (size 0.8) (drill 0.4) (layers F.Cu B.Cu) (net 5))
 (segment (start 207.5 65.4) (end 207.5 69.9) (width 0.25) (layer F.Cu) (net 5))
 (segment (start 203.74 69.26) (end 203.74 73.5) (width 0.25) (layer B.Cu) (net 5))
 (segment (start 204.3 68.7) (end 203.74 69.26) (width 0.25) (layer B.Cu) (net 5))
 (segment (start 206.3 68.7) (end 204.3 68.7) (width 0.25) (layer B.Cu) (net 5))
 (segment (start 207.5 69.9) (end 206.3 68.7) (width 0.25) (layer B.Cu) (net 5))
 (via (at 207.6 77.599996) (size 0.8) (drill 0.4) (layers F.Cu B.Cu) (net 5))
 (segment (start 207.56 77.559996) (end 207.6 77.599996) (width 0.25) (layer B.Cu) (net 5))
 (segment (start 207.56 69.96) (end 207.56 77.559996) (width 0.25) (layer B.Cu) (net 5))
 (segment (start 207.5 69.9) (end 207.56 69.96) (width 0.25) (layer B.Cu) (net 5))
 (via (at 207.4 92.1) (size 0.8) (drill 0.4) (layers F.Cu B.Cu) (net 5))
 (segment (start 207.5 95.5) (end 207.5 92.2) (width 0.25) (layer B.Cu) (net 5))
 (segment (start 207.5 92.2) (end 207.4 92.1) (width 0.25) (layer B.Cu) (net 5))
 (segment (start 207.6 77.599996) (end 207.6 91.9) (width 0.25) (layer F.Cu) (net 5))
 (segment (start 207.6 91.9) (end 207.4 92.1) (width 0.25) (layer F.Cu) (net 5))
 (via (at 204.7 65.4) (size 0.8) (drill 0.4) (layers F.Cu B.Cu) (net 6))
 (segment (start 204.73 65.37) (end 204.7 65.4) (width 0.25) (layer B.Cu) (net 6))
 (segment (start 204.73 62.5) (end 204.73 65.37) (width 0.25) (layer B.Cu) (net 6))
 (via (at 204.7 69.9) (size 0.8) (drill 0.4) (layers F.Cu B.Cu) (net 6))
 (segment (start 204.7 65.4) (end 204.7 69.9) (width 0.25) (layer F.Cu) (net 6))
 (segment (start 204.7 70.9) (end 206.28 72.48) (width 0.25) (layer B.Cu) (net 6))
 (segment (start 206.28 72.48) (end 206.28 73.5) (width 0.25) (layer B.Cu) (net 6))
 (segment (start 204.7 69.9) (end 204.7 70.9) (width 0.25) (layer B.Cu) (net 6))
 (via (at 203.7 77.6) (size 0.8) (drill 0.4) (layers F.Cu B.Cu) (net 6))
 (segment (start 206.28 73.5) (end 206.28 75.02) (width 0.25) (layer B.Cu) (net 6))
 (segment (start 206.28 75.02) (end 203.7 77.6) (width 0.25) (layer B.Cu) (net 6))
 (via (at 204.6 92.1) (size 0.8) (drill 0.4) (layers F.Cu B.Cu) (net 6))
 (segment (start 204.73 95.5) (end 204.73 92.23) (width 0.25) (layer B.Cu) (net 6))
 (segment (start 204.73 92.23) (end 204.6 92.1) (width 0.25) (layer B.Cu) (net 6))
 (segment (start 203.7 77.6) (end 203.7 91.2) (width 0.25) (layer F.Cu) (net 6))
 (segment (start 203.7 91.2) (end 204.6 92.1) (width 0.25) (layer F.Cu) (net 6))
 (via (at 202 65.4) (size 0.8) (drill 0.4) (layers F.Cu B.Cu) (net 19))
 (segment (start 201.96 65.36) (end 202 65.4) (width 0.25) (layer B.Cu) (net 19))
 (segment (start 201.96 62.5) (end 201.96 65.36) (width 0.25) (layer B.Cu) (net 19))
 (segment (start 201.1 66.3) (end 201.1 69.9) (width 0.25) (layer F.Cu) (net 19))
 (segment (start 202 65.4) (end 201.1 66.3) (width 0.25) (layer F.Cu) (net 19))
 (via (at 201.1 69.9) (size 0.8) (drill 0.4) (layers F.Cu B.Cu) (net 19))
 (via (at 201.3 77.59999) (size 0.8) (drill 0.4) (layers F.Cu B.Cu) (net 19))
 (segment (start 202.48 76.41999) (end 201.3 77.59999) (width 0.25) (layer B.Cu) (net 19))
 (segment (start 202.48 71.28) (end 202.48 76.41999) (width 0.25) (layer B.Cu) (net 19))
 (segment (start 201.1 69.9) (end 202.48 71.28) (width 0.25) (layer B.Cu) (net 19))
 (via (at 201.800001 92.099999) (size 0.8) (drill 0.4) (layers F.Cu B.Cu) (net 19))
 (segment (start 201.3 91.599998) (end 201.800001 92.099999) (width 0.25) (layer F.Cu) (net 19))
 (segment (start 201.96 92.259998) (end 201.800001 92.099999) (width 0.25) (layer B.Cu) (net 19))
 (segment (start 201.96 95.5) (end 201.96 92.259998) (width 0.25) (layer B.Cu) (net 19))
 (segment (start 201.3 77.59999) (end 201.3 91.599998) (width 0.25) (layer F.Cu) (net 19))
 (via (at 199.2 65.4) (size 0.8) (drill 0.4) (layers F.Cu B.Cu) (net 8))
 (segment (start 199.19 65.39) (end 199.2 65.4) (width 0.25) (layer B.Cu) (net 8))
 (segment (start 199.19 62.5) (end 199.19 65.39) (width 0.25) (layer B.Cu) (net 8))
 (via (at 198.8 82.5) (size 0.8) (drill 0.4) (layers F.Cu B.Cu) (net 8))
 (segment (start 198.8 82.5) (end 211.7 82.5) (width 0.25) (layer B.Cu) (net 8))
 (segment (start 211.7 82.5) (end 214.7 79.5) (width 0.25) (layer B.Cu) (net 8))
 (segment (start 214.7 79.5) (end 214.7 77.4) (width 0.25) (layer B.Cu) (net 8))
 (segment (start 216.44 75.66) (end 216.44 73.5) (width 0.25) (layer B.Cu) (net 8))
 (segment (start 214.7 77.4) (end 216.44 75.66) (width 0.25) (layer B.Cu) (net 8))
 (via (at 199.20001 69.9) (size 0.8) (drill 0.4) (layers F.Cu B.Cu) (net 8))
 (segment (start 199.2 65.4) (end 199.2 69.89999) (width 0.25) (layer F.Cu) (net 8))
 (segment (start 199.2 69.89999) (end 199.20001 69.9) (width 0.25) (layer F.Cu) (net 8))
 (segment (start 198.8 82.5) (end 198.8 77.599996) (width 0.25) (layer F.Cu) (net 8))
 (via (at 198.8 77.599996) (size 0.8) (drill 0.4) (layers F.Cu B.Cu) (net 8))
 (segment (start 199.93 76.469996) (end 198.8 77.599996) (width 0.25) (layer B.Cu) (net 8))
 (segment (start 199.93 70.62999) (end 199.93 76.469996) (width 0.25) (layer B.Cu) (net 8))
 (segment (start 199.20001 69.9) (end 199.93 70.62999) (width 0.25) (layer B.Cu) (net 8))
 (via (at 199.050001 92.150001) (size 0.8) (drill 0.4) (layers F.Cu B.Cu) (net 8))
 (segment (start 199.19 92.29) (end 199.050001 92.150001) (width 0.25) (layer B.Cu) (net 8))
 (segment (start 198.8 82.5) (end 198.8 91.9) (width 0.25) (layer F.Cu) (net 8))
 (segment (start 198.8 91.9) (end 199.050001 92.150001) (width 0.25) (layer F.Cu) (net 8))
 (segment (start 199.19 95.5) (end 199.19 92.29) (width 0.25) (layer B.Cu) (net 8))
 (segment (start 196.42 65.38) (end 196.4 65.4) (width 0.25) (layer B.Cu) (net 18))
 (via (at 196.4 65.4) (size 0.8) (drill 0.4) (layers F.Cu B.Cu) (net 18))
 (segment (start 196.42 62.5) (end 196.42 65.38) (width 0.25) (layer B.Cu) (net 18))
 (segment (start 196.4 65.4) (end 196.4 70.1) (width 0.25) (layer F.Cu) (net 18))
 (via (at 196.4 69.900008) (size 0.8) (drill 0.4) (layers F.Cu B.Cu) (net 18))
 (segment (start 196.4 70.1) (end 196.4 69.900008) (width 0.25) (layer F.Cu) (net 18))
 (segment (start 197.4 70.900008) (end 197.4 76.4) (width 0.25) (layer B.Cu) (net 18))
 (segment (start 196.4 69.900008) (end 197.4 70.900008) (width 0.25) (layer B.Cu) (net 18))
 (via (at 196.2 77.6) (size 0.8) (drill 0.4) (layers F.Cu B.Cu) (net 18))
 (segment (start 197.4 76.4) (end 196.2 77.6) (width 0.25) (layer B.Cu) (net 18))
 (segment (start 196.2 91.8) (end 196.5 92.1) (width 0.25) (layer F.Cu) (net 18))
 (segment (start 196.2 77.6) (end 196.2 91.8) (width 0.25) (layer F.Cu) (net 18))
 (segment (start 196.42 92.18) (end 196.5 92.1) (width 0.25) (layer B.Cu) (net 18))
 (segment (start 196.42 95.5) (end 196.42 92.18) (width 0.25) (layer B.Cu) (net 18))
 (via (at 196.5 92.1) (size 0.8) (drill 0.4) (layers F.Cu B.Cu) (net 18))
 (via (at 193.7 65.4) (size 0.8) (drill 0.4) (layers F.Cu B.Cu) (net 17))
 (segment (start 193.65 65.35) (end 193.7 65.4) (width 0.25) (layer B.Cu) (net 17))
 (segment (start 193.65 62.5) (end 193.65 65.35) (width 0.25) (layer B.Cu) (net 17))
 (segment (start 193.7 65.4) (end 193.7 69.9) (width 0.25) (layer F.Cu) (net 17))
 (via (at 193.7 69.9) (size 0.8) (drill 0.4) (layers F.Cu B.Cu) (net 17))
 (via (at 193.7 77.600008) (size 0.8) (drill 0.4) (layers F.Cu B.Cu) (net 17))
 (segment (start 194.85 76.450008) (end 193.7 77.600008) (width 0.25) (layer B.Cu) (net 17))
 (segment (start 194.85 71.05) (end 194.85 76.450008) (width 0.25) (layer B.Cu) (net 17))
 (segment (start 193.7 69.9) (end 194.85 71.05) (width 0.25) (layer B.Cu) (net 17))
 (via (at 193.7 92.100004) (size 0.8) (drill 0.4) (layers F.Cu B.Cu) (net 17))
 (segment (start 193.7 77.600008) (end 193.7 92.100004) (width 0.25) (layer F.Cu) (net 17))
 (segment (start 193.65 95.5) (end 193.65 92.150004) (width 0.25) (layer B.Cu) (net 17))
 (segment (start 193.65 92.150004) (end 193.7 92.100004) (width 0.25) (layer B.Cu) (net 17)))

